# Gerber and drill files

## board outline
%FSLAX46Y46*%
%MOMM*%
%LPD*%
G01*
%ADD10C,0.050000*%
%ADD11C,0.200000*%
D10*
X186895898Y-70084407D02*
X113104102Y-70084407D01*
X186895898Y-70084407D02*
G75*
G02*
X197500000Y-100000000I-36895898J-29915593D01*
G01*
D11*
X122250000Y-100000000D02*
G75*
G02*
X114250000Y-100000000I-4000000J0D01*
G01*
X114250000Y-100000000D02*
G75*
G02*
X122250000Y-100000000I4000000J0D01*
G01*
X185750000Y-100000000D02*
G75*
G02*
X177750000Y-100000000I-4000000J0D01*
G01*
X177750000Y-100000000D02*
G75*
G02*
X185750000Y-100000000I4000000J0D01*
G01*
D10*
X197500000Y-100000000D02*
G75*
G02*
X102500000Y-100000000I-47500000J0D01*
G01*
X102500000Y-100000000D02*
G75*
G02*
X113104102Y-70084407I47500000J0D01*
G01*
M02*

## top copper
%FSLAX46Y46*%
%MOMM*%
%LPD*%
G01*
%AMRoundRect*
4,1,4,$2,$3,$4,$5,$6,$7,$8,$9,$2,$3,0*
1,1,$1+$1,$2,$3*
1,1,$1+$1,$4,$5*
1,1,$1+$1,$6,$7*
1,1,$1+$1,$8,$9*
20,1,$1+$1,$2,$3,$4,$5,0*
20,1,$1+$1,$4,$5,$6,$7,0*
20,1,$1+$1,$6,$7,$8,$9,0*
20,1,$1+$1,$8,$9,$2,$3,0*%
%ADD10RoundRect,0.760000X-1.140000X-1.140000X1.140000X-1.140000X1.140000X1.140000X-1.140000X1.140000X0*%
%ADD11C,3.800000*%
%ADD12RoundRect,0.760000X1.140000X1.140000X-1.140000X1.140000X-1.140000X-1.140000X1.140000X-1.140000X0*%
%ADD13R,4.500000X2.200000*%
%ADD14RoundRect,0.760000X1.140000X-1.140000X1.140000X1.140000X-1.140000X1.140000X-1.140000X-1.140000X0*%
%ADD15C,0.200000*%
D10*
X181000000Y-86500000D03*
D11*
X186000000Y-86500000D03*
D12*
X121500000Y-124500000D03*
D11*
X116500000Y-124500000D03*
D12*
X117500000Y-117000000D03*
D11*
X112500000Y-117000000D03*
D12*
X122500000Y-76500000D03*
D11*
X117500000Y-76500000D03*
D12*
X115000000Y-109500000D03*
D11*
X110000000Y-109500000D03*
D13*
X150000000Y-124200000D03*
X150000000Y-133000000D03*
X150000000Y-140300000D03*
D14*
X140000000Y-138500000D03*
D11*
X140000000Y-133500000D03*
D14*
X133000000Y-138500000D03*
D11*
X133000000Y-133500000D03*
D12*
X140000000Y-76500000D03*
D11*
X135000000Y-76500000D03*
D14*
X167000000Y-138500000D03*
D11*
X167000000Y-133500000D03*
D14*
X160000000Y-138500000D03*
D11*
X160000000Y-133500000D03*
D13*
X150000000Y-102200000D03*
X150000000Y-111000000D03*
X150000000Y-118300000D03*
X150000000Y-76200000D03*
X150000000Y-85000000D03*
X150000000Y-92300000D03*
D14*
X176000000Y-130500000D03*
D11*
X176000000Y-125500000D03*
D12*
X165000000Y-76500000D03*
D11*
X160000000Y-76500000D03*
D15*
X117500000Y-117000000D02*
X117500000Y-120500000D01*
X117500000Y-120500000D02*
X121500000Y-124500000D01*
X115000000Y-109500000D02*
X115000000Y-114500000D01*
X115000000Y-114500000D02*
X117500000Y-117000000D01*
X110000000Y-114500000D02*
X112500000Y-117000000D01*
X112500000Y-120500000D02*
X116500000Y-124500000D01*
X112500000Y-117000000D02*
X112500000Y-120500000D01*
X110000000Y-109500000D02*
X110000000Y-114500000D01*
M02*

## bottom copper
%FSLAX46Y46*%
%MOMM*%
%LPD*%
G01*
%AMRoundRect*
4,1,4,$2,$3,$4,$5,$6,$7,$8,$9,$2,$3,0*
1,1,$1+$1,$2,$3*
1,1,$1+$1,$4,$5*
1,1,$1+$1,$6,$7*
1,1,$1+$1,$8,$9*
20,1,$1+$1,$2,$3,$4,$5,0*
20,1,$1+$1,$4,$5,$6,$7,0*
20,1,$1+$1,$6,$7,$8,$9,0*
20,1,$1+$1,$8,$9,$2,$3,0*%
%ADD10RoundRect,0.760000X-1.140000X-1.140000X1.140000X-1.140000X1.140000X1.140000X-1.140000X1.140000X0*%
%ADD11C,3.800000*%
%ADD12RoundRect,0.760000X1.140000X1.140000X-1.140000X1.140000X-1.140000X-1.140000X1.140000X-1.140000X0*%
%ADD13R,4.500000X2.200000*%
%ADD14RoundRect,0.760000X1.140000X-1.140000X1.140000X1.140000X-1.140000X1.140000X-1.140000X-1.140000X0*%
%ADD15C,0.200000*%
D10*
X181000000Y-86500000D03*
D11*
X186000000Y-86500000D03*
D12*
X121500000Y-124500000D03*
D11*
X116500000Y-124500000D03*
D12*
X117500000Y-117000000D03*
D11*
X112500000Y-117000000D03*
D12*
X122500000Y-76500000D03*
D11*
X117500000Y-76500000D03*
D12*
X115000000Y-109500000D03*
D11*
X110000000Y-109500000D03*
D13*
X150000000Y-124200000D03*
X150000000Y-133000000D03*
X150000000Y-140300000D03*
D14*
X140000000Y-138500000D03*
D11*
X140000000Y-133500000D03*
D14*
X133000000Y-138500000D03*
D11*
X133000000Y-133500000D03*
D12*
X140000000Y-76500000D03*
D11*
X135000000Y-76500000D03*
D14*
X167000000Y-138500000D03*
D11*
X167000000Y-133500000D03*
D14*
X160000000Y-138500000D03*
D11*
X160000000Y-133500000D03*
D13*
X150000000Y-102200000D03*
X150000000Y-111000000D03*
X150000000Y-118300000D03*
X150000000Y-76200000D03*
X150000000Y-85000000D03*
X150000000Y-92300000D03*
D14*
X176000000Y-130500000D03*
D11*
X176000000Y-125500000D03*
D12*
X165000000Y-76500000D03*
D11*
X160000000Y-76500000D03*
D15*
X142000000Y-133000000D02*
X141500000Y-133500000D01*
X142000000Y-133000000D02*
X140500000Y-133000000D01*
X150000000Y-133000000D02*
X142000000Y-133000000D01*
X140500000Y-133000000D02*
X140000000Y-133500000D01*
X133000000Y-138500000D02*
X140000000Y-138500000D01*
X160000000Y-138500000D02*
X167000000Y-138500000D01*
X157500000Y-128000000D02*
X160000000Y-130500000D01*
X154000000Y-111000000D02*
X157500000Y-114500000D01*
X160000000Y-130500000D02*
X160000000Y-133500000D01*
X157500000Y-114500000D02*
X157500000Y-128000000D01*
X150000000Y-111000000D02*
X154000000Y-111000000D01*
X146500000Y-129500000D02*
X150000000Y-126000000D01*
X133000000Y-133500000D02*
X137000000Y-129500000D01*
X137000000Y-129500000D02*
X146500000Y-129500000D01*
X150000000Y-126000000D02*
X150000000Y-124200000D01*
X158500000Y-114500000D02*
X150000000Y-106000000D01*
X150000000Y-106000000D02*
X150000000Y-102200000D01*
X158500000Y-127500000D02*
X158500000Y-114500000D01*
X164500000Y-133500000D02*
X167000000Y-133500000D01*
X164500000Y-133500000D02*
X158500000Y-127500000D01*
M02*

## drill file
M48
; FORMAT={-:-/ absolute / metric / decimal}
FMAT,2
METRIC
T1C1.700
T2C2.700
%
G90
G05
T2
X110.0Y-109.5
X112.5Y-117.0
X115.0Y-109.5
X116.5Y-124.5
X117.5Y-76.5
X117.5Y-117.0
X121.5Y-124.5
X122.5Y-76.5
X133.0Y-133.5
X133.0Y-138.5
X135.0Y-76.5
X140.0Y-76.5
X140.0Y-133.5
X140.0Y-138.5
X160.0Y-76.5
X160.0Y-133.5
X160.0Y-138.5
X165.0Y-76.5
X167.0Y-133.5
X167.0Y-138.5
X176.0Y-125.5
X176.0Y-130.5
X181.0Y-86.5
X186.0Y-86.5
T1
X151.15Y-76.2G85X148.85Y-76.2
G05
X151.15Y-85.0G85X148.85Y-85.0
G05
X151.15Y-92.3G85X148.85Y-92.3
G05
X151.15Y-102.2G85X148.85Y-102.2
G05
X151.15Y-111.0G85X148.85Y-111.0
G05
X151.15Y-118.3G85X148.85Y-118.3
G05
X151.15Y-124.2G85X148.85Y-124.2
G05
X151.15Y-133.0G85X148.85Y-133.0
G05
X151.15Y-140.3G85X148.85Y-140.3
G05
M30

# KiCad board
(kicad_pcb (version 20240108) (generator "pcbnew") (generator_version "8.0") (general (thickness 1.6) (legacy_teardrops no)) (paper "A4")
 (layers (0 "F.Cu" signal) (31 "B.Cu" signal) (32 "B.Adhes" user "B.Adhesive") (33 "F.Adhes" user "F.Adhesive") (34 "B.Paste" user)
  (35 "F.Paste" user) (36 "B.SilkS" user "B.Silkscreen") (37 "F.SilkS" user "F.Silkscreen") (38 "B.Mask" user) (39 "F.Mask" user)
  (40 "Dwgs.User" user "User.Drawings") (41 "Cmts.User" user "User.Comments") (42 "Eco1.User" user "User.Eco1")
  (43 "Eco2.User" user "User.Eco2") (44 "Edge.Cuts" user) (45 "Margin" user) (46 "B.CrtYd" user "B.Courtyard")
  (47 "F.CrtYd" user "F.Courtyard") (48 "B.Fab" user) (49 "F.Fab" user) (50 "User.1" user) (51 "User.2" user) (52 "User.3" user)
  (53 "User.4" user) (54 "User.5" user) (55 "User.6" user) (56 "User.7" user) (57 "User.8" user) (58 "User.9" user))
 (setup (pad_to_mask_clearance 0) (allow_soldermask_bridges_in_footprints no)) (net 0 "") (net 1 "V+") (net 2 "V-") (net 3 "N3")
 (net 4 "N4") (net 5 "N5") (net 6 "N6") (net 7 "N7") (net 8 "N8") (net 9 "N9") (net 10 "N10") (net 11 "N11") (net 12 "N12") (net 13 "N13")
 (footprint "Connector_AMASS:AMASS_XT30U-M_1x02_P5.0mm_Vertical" (layer "F.Cu") (at 181 86.5)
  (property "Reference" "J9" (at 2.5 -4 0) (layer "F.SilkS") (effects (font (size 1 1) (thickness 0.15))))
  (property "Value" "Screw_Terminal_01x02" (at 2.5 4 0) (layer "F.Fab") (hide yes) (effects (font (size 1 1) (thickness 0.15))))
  (pad "1" thru_hole roundrect (at 0 0) (size 3.8 3.8) (drill 2.7) (layers "*.Cu" "*.Mask") (remove_unused_layers no) (roundrect_rratio 0.2)
   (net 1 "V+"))
  (pad "2" thru_hole circle (at 5 0) (size 3.8 3.8) (drill 2.7) (layers "*.Cu" "*.Mask") (remove_unused_layers no) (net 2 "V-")))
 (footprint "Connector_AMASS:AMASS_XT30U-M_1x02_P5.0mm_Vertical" (layer "F.Cu") (at 121.5 124.5 180)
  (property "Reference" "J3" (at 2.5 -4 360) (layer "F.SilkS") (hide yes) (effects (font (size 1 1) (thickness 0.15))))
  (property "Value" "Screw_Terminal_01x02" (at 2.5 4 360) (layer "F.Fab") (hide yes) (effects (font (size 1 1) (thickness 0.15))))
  (pad "1" thru_hole roundrect (at 0 0 180) (size 3.8 3.8) (drill 2.7) (layers "*.Cu" "*.Mask") (remove_unused_layers no)
   (roundrect_rratio 0.2) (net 2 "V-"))
  (pad "2" thru_hole circle (at 5 0 180) (size 3.8 3.8) (drill 2.7) (layers "*.Cu" "*.Mask") (remove_unused_layers no) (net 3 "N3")))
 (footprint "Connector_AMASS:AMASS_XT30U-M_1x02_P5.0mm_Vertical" (layer "F.Cu") (at 117.5 117 180)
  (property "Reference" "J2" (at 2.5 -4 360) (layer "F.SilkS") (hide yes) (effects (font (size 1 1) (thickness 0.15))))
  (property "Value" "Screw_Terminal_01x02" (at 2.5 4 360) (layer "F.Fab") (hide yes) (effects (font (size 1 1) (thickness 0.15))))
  (pad "1" thru_hole roundrect (at 0 0 180) (size 3.8 3.8) (drill 2.7) (layers "*.Cu" "*.Mask") (remove_unused_layers no)
   (roundrect_rratio 0.2) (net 2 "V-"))
  (pad "2" thru_hole circle (at 5 0 180) (size 3.8 3.8) (drill 2.7) (layers "*.Cu" "*.Mask") (remove_unused_layers no) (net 3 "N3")))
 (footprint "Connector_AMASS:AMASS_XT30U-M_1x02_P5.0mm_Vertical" (layer "F.Cu") (at 122.5 76.5 180)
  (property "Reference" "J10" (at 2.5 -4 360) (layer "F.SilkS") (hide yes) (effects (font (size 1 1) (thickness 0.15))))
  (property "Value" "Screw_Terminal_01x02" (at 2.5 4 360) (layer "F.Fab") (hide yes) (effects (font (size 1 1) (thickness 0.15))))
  (pad "1" thru_hole roundrect (at 0 0 180) (size 3.8 3.8) (drill 2.7) (layers "*.Cu" "*.Mask") (remove_unused_layers no)
   (roundrect_rratio 0.2) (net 1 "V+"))
  (pad "2" thru_hole circle (at 5 0 180) (size 3.8 3.8) (drill 2.7) (layers "*.Cu" "*.Mask") (remove_unused_layers no) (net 2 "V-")))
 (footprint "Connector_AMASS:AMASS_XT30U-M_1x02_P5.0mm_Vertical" (layer "F.Cu") (at 115 109.5 180)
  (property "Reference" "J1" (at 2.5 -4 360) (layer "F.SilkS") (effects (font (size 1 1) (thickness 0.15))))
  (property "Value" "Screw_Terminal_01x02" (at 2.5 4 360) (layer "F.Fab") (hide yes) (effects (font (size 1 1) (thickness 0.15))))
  (pad "1" thru_hole roundrect (at 0 0 180) (size 3.8 3.8) (drill 2.7) (layers "*.Cu" "*.Mask") (remove_unused_layers no)
   (roundrect_rratio 0.2) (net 2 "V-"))
  (pad "2" thru_hole circle (at 5 0 180) (size 3.8 3.8) (drill 2.7) (layers "*.Cu" "*.Mask") (remove_unused_layers no) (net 3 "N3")))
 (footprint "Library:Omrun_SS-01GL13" (layer "B.Cu") (at 150 133 -90)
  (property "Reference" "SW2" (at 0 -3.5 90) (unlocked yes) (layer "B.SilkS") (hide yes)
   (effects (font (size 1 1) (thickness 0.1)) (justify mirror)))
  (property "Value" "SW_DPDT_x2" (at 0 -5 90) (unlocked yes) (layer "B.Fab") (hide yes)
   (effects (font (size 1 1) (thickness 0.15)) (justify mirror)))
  (pad "1" thru_hole rect (at -8.8 0 270) (size 2.2 4.5) (drill oval 1.7 4) (layers "*.Cu" "*.Mask") (remove_unused_layers no) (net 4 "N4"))
  (pad "2" thru_hole rect (at 0 0 270) (size 2.2 4.5) (drill oval 1.7 4) (layers "*.Cu" "*.Mask") (remove_unused_layers no) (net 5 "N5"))
  (pad "3" thru_hole rect (at 7.3 0 270) (size 2.2 4.5) (drill oval 1.7 4) (layers "*.Cu" "*.Mask") (remove_unused_layers no) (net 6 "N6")))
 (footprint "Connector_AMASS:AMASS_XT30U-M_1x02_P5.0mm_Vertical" (layer "B.Cu") (at 140 138.5 90)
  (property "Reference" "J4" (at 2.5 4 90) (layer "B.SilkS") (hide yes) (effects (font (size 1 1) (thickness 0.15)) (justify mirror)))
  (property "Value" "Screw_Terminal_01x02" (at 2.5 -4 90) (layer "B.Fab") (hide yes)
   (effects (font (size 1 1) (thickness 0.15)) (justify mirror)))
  (pad "1" thru_hole roundrect (at 0 0 90) (size 3.8 3.8) (drill 2.7) (layers "*.Cu" "*.Mask") (remove_unused_layers no)
   (roundrect_rratio 0.2) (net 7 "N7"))
  (pad "2" thru_hole circle (at 5 0 90) (size 3.8 3.8) (drill 2.7) (layers "*.Cu" "*.Mask") (remove_unused_layers no) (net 5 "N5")))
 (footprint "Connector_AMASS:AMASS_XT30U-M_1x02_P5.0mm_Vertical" (layer "B.Cu") (at 133 138.5 90)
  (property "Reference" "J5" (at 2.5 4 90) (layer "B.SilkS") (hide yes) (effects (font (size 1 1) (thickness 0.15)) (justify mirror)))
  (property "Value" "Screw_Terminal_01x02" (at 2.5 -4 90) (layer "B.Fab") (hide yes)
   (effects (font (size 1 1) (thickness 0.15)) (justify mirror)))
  (pad "1" thru_hole roundrect (at 0 0 90) (size 3.8 3.8) (drill 2.7) (layers "*.Cu" "*.Mask") (remove_unused_layers no)
   (roundrect_rratio 0.2) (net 7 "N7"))
  (pad "2" thru_hole circle (at 5 0 90) (size 3.8 3.8) (drill 2.7) (layers "*.Cu" "*.Mask") (remove_unused_layers no) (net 4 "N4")))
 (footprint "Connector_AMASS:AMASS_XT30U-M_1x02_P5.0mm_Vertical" (layer "B.Cu") (at 140 76.5 180)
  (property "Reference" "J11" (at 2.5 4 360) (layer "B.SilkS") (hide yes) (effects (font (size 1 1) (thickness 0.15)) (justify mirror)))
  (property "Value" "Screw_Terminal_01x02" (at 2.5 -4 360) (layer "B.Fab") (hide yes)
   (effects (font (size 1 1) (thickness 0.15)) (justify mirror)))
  (pad "1" thru_hole roundrect (at 0 0 180) (size 3.8 3.8) (drill 2.7) (layers "*.Cu" "*.Mask") (remove_unused_layers no)
   (roundrect_rratio 0.2) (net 1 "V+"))
  (pad "2" thru_hole circle (at 5 0 180) (size 3.8 3.8) (drill 2.7) (layers "*.Cu" "*.Mask") (remove_unused_layers no) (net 2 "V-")))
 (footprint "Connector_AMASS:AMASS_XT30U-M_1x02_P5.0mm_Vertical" (layer "B.Cu") (at 167 138.5 90)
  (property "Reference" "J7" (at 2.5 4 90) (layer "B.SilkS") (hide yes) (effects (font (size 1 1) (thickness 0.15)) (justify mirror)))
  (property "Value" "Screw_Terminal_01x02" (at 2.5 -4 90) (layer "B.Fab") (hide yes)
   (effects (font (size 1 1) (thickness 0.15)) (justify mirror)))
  (pad "1" thru_hole roundrect (at 0 0 90) (size 3.8 3.8) (drill 2.7) (layers "*.Cu" "*.Mask") (remove_unused_layers no)
   (roundrect_rratio 0.2) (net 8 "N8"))
  (pad "2" thru_hole circle (at 5 0 90) (size 3.8 3.8) (drill 2.7) (layers "*.Cu" "*.Mask") (remove_unused_layers no) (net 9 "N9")))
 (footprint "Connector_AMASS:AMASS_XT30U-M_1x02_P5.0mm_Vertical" (layer "B.Cu") (at 160 138.5 90)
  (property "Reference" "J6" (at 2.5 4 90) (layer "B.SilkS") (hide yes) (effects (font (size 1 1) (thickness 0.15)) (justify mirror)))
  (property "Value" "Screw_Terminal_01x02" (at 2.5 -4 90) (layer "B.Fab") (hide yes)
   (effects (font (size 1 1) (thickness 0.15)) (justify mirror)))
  (pad "1" thru_hole roundrect (at 0 0 90) (size 3.8 3.8) (drill 2.7) (layers "*.Cu" "*.Mask") (remove_unused_layers no)
   (roundrect_rratio 0.2) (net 8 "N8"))
  (pad "2" thru_hole circle (at 5 0 90) (size 3.8 3.8) (drill 2.7) (layers "*.Cu" "*.Mask") (remove_unused_layers no) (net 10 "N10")))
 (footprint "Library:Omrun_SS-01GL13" (layer "B.Cu") (at 150 111 -90)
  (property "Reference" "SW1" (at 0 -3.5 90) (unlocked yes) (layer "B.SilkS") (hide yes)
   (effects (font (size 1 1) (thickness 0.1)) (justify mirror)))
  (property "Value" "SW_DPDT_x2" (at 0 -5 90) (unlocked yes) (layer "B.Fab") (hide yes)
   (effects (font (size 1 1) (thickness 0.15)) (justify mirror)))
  (pad "1" thru_hole rect (at -8.8 0 270) (size 2.2 4.5) (drill oval 1.7 4) (layers "*.Cu" "*.Mask") (remove_unused_layers no) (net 9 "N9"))
  (pad "2" thru_hole rect (at 0 0 270) (size 2.2 4.5) (drill oval 1.7 4) (layers "*.Cu" "*.Mask") (remove_unused_layers no) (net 10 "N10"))
  (pad "3" thru_hole rect (at 7.3 0 270) (size 2.2 4.5) (drill oval 1.7 4) (layers "*.Cu" "*.Mask") (remove_unused_layers no) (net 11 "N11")))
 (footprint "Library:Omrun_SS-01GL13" (layer "B.Cu") (at 150 85 -90)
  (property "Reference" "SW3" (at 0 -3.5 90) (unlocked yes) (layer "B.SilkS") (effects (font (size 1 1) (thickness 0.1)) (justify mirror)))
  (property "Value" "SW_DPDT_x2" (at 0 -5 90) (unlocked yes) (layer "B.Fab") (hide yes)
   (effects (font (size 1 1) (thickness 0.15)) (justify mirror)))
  (pad "1" thru_hole rect (at -8.8 0 270) (size 2.2 4.5) (drill oval 1.7 4) (layers "*.Cu" "*.Mask") (remove_unused_layers no)
   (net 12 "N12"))
  (pad "2" thru_hole rect (at 0 0 270) (size 2.2 4.5) (drill oval 1.7 4) (layers "*.Cu" "*.Mask") (remove_unused_layers no) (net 3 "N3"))
  (pad "3" thru_hole rect (at 7.3 0 270) (size 2.2 4.5) (drill oval 1.7 4) (layers "*.Cu" "*.Mask") (remove_unused_layers no) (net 1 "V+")))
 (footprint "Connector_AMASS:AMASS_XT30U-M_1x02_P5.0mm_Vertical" (layer "B.Cu") (at 176 130.5 90)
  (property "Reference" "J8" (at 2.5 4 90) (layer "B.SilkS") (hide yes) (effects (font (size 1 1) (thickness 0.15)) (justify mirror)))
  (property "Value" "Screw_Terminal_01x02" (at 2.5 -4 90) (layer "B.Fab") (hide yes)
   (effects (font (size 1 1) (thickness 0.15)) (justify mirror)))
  (pad "1" thru_hole roundrect (at 0 0 90) (size 3.8 3.8) (drill 2.7) (layers "*.Cu" "*.Mask") (remove_unused_layers no)
   (roundrect_rratio 0.2) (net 1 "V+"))
  (pad "2" thru_hole circle (at 5 0 90) (size 3.8 3.8) (drill 2.7) (layers "*.Cu" "*.Mask") (remove_unused_layers no) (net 2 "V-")))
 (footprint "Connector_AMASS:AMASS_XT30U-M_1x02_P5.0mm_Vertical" (layer "B.Cu") (at 165 76.5 180)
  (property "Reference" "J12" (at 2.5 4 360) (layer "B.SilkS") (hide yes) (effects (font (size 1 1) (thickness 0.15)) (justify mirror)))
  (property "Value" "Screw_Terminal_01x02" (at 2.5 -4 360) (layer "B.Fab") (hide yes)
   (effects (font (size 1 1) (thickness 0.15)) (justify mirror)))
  (pad "1" thru_hole roundrect (at 0 0 180) (size 3.8 3.8) (drill 2.7) (layers "*.Cu" "*.Mask") (remove_unused_layers no)
   (roundrect_rratio 0.2) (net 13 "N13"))
  (pad "2" thru_hole circle (at 5 0 180) (size 3.8 3.8) (drill 2.7) (layers "*.Cu" "*.Mask") (remove_unused_layers no) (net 2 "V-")))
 (gr_line (start 186.895898 70.084407) (end 113.104102 70.084407) (stroke (width 0.05) (type default)) (layer "Edge.Cuts"))
 (gr_arc (start 186.895898 70.084407) (mid 194.770555 84.130299) (end 197.5 100) (stroke (width 0.05) (type default)) (layer "Edge.Cuts"))
 (gr_circle (center 118.25 100) (end 122.25 100) (stroke (width 0.2) (type default)) (fill none) (layer "Edge.Cuts"))
 (gr_circle (center 181.75 100) (end 185.75 100) (stroke (width 0.2) (type default)) (fill none) (layer "Edge.Cuts"))
 (gr_arc (start 197.5 100) (mid 150 147.5) (end 102.5 100) (stroke (width 0.05) (type default)) (layer "Edge.Cuts"))
 (gr_arc (start 102.5 100) (mid 105.229445 84.130299) (end 113.104102 70.084407) (stroke (width 0.05) (type default)) (layer "Edge.Cuts"))
 (segment (start 117.5 117) (end 117.5 120.5) (width 0.2) (layer "F.Cu") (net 2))
 (segment (start 117.5 120.5) (end 121.5 124.5) (width 0.2) (layer "F.Cu") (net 2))
 (segment (start 115 109.5) (end 115 114.5) (width 0.2) (layer "F.Cu") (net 2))
 (segment (start 115 114.5) (end 117.5 117) (width 0.2) (layer "F.Cu") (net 2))
 (segment (start 110 114.5) (end 112.5 117) (width 0.2) (layer "F.Cu") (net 3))
 (segment (start 112.5 120.5) (end 116.5 124.5) (width 0.2) (layer "F.Cu") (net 3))
 (segment (start 112.5 117) (end 112.5 120.5) (width 0.2) (layer "F.Cu") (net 3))
 (segment (start 110 109.5) (end 110 114.5) (width 0.2) (layer "F.Cu") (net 3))
 (segment (start 142 133) (end 141.5 133.5) (width 0.2) (layer "B.Cu") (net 5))
 (segment (start 142 133) (end 140.5 133) (width 0.2) (layer "B.Cu") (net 5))
 (segment (start 150 133) (end 142 133) (width 0.2) (layer "B.Cu") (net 5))
 (segment (start 140.5 133) (end 140 133.5) (width 0.2) (layer "B.Cu") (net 5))
 (segment (start 133 138.5) (end 140 138.5) (width 0.2) (layer "B.Cu") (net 7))
 (segment (start 160 138.5) (end 167 138.5) (width 0.2) (layer "B.Cu") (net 8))
 (segment (start 157.5 128) (end 160 130.5) (width 0.2) (layer "B.Cu") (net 10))
 (segment (start 154 111) (end 157.5 114.5) (width 0.2) (layer "B.Cu") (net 10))
 (segment (start 160 130.5) (end 160 133.5) (width 0.2) (layer "B.Cu") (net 10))
 (segment (start 157.5 114.5) (end 157.5 128) (width 0.2) (layer "B.Cu") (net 10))
 (segment (start 150 111) (end 154 111) (width 0.2) (layer "B.Cu") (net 10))
 (segment (start 146.5 129.5) (end 150 126) (width 0.2) (layer "B.Cu") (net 4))
 (segment (start 133 133.5) (end 137 129.5) (width 0.2) (layer "B.Cu") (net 4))
 (segment (start 137 129.5) (end 146.5 129.5) (width 0.2) (layer "B.Cu") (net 4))
 (segment (start 150 126) (end 150 124.2) (width 0.2) (layer "B.Cu") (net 4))
 (segment (start 158.5 114.5) (end 150 106) (width 0.2) (layer "B.Cu") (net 9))
 (segment (start 150 106) (end 150 102.2) (width 0.2) (layer "B.Cu") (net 9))
 (segment (start 158.5 127.5) (end 158.5 114.5) (width 0.2) (layer "B.Cu") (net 9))
 (segment (start 164.5 133.5) (end 167 133.5) (width 0.2) (layer "B.Cu") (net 9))
 (segment (start 164.5 133.5) (end 158.5 127.5) (width 0.2) (layer "B.Cu") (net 9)))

